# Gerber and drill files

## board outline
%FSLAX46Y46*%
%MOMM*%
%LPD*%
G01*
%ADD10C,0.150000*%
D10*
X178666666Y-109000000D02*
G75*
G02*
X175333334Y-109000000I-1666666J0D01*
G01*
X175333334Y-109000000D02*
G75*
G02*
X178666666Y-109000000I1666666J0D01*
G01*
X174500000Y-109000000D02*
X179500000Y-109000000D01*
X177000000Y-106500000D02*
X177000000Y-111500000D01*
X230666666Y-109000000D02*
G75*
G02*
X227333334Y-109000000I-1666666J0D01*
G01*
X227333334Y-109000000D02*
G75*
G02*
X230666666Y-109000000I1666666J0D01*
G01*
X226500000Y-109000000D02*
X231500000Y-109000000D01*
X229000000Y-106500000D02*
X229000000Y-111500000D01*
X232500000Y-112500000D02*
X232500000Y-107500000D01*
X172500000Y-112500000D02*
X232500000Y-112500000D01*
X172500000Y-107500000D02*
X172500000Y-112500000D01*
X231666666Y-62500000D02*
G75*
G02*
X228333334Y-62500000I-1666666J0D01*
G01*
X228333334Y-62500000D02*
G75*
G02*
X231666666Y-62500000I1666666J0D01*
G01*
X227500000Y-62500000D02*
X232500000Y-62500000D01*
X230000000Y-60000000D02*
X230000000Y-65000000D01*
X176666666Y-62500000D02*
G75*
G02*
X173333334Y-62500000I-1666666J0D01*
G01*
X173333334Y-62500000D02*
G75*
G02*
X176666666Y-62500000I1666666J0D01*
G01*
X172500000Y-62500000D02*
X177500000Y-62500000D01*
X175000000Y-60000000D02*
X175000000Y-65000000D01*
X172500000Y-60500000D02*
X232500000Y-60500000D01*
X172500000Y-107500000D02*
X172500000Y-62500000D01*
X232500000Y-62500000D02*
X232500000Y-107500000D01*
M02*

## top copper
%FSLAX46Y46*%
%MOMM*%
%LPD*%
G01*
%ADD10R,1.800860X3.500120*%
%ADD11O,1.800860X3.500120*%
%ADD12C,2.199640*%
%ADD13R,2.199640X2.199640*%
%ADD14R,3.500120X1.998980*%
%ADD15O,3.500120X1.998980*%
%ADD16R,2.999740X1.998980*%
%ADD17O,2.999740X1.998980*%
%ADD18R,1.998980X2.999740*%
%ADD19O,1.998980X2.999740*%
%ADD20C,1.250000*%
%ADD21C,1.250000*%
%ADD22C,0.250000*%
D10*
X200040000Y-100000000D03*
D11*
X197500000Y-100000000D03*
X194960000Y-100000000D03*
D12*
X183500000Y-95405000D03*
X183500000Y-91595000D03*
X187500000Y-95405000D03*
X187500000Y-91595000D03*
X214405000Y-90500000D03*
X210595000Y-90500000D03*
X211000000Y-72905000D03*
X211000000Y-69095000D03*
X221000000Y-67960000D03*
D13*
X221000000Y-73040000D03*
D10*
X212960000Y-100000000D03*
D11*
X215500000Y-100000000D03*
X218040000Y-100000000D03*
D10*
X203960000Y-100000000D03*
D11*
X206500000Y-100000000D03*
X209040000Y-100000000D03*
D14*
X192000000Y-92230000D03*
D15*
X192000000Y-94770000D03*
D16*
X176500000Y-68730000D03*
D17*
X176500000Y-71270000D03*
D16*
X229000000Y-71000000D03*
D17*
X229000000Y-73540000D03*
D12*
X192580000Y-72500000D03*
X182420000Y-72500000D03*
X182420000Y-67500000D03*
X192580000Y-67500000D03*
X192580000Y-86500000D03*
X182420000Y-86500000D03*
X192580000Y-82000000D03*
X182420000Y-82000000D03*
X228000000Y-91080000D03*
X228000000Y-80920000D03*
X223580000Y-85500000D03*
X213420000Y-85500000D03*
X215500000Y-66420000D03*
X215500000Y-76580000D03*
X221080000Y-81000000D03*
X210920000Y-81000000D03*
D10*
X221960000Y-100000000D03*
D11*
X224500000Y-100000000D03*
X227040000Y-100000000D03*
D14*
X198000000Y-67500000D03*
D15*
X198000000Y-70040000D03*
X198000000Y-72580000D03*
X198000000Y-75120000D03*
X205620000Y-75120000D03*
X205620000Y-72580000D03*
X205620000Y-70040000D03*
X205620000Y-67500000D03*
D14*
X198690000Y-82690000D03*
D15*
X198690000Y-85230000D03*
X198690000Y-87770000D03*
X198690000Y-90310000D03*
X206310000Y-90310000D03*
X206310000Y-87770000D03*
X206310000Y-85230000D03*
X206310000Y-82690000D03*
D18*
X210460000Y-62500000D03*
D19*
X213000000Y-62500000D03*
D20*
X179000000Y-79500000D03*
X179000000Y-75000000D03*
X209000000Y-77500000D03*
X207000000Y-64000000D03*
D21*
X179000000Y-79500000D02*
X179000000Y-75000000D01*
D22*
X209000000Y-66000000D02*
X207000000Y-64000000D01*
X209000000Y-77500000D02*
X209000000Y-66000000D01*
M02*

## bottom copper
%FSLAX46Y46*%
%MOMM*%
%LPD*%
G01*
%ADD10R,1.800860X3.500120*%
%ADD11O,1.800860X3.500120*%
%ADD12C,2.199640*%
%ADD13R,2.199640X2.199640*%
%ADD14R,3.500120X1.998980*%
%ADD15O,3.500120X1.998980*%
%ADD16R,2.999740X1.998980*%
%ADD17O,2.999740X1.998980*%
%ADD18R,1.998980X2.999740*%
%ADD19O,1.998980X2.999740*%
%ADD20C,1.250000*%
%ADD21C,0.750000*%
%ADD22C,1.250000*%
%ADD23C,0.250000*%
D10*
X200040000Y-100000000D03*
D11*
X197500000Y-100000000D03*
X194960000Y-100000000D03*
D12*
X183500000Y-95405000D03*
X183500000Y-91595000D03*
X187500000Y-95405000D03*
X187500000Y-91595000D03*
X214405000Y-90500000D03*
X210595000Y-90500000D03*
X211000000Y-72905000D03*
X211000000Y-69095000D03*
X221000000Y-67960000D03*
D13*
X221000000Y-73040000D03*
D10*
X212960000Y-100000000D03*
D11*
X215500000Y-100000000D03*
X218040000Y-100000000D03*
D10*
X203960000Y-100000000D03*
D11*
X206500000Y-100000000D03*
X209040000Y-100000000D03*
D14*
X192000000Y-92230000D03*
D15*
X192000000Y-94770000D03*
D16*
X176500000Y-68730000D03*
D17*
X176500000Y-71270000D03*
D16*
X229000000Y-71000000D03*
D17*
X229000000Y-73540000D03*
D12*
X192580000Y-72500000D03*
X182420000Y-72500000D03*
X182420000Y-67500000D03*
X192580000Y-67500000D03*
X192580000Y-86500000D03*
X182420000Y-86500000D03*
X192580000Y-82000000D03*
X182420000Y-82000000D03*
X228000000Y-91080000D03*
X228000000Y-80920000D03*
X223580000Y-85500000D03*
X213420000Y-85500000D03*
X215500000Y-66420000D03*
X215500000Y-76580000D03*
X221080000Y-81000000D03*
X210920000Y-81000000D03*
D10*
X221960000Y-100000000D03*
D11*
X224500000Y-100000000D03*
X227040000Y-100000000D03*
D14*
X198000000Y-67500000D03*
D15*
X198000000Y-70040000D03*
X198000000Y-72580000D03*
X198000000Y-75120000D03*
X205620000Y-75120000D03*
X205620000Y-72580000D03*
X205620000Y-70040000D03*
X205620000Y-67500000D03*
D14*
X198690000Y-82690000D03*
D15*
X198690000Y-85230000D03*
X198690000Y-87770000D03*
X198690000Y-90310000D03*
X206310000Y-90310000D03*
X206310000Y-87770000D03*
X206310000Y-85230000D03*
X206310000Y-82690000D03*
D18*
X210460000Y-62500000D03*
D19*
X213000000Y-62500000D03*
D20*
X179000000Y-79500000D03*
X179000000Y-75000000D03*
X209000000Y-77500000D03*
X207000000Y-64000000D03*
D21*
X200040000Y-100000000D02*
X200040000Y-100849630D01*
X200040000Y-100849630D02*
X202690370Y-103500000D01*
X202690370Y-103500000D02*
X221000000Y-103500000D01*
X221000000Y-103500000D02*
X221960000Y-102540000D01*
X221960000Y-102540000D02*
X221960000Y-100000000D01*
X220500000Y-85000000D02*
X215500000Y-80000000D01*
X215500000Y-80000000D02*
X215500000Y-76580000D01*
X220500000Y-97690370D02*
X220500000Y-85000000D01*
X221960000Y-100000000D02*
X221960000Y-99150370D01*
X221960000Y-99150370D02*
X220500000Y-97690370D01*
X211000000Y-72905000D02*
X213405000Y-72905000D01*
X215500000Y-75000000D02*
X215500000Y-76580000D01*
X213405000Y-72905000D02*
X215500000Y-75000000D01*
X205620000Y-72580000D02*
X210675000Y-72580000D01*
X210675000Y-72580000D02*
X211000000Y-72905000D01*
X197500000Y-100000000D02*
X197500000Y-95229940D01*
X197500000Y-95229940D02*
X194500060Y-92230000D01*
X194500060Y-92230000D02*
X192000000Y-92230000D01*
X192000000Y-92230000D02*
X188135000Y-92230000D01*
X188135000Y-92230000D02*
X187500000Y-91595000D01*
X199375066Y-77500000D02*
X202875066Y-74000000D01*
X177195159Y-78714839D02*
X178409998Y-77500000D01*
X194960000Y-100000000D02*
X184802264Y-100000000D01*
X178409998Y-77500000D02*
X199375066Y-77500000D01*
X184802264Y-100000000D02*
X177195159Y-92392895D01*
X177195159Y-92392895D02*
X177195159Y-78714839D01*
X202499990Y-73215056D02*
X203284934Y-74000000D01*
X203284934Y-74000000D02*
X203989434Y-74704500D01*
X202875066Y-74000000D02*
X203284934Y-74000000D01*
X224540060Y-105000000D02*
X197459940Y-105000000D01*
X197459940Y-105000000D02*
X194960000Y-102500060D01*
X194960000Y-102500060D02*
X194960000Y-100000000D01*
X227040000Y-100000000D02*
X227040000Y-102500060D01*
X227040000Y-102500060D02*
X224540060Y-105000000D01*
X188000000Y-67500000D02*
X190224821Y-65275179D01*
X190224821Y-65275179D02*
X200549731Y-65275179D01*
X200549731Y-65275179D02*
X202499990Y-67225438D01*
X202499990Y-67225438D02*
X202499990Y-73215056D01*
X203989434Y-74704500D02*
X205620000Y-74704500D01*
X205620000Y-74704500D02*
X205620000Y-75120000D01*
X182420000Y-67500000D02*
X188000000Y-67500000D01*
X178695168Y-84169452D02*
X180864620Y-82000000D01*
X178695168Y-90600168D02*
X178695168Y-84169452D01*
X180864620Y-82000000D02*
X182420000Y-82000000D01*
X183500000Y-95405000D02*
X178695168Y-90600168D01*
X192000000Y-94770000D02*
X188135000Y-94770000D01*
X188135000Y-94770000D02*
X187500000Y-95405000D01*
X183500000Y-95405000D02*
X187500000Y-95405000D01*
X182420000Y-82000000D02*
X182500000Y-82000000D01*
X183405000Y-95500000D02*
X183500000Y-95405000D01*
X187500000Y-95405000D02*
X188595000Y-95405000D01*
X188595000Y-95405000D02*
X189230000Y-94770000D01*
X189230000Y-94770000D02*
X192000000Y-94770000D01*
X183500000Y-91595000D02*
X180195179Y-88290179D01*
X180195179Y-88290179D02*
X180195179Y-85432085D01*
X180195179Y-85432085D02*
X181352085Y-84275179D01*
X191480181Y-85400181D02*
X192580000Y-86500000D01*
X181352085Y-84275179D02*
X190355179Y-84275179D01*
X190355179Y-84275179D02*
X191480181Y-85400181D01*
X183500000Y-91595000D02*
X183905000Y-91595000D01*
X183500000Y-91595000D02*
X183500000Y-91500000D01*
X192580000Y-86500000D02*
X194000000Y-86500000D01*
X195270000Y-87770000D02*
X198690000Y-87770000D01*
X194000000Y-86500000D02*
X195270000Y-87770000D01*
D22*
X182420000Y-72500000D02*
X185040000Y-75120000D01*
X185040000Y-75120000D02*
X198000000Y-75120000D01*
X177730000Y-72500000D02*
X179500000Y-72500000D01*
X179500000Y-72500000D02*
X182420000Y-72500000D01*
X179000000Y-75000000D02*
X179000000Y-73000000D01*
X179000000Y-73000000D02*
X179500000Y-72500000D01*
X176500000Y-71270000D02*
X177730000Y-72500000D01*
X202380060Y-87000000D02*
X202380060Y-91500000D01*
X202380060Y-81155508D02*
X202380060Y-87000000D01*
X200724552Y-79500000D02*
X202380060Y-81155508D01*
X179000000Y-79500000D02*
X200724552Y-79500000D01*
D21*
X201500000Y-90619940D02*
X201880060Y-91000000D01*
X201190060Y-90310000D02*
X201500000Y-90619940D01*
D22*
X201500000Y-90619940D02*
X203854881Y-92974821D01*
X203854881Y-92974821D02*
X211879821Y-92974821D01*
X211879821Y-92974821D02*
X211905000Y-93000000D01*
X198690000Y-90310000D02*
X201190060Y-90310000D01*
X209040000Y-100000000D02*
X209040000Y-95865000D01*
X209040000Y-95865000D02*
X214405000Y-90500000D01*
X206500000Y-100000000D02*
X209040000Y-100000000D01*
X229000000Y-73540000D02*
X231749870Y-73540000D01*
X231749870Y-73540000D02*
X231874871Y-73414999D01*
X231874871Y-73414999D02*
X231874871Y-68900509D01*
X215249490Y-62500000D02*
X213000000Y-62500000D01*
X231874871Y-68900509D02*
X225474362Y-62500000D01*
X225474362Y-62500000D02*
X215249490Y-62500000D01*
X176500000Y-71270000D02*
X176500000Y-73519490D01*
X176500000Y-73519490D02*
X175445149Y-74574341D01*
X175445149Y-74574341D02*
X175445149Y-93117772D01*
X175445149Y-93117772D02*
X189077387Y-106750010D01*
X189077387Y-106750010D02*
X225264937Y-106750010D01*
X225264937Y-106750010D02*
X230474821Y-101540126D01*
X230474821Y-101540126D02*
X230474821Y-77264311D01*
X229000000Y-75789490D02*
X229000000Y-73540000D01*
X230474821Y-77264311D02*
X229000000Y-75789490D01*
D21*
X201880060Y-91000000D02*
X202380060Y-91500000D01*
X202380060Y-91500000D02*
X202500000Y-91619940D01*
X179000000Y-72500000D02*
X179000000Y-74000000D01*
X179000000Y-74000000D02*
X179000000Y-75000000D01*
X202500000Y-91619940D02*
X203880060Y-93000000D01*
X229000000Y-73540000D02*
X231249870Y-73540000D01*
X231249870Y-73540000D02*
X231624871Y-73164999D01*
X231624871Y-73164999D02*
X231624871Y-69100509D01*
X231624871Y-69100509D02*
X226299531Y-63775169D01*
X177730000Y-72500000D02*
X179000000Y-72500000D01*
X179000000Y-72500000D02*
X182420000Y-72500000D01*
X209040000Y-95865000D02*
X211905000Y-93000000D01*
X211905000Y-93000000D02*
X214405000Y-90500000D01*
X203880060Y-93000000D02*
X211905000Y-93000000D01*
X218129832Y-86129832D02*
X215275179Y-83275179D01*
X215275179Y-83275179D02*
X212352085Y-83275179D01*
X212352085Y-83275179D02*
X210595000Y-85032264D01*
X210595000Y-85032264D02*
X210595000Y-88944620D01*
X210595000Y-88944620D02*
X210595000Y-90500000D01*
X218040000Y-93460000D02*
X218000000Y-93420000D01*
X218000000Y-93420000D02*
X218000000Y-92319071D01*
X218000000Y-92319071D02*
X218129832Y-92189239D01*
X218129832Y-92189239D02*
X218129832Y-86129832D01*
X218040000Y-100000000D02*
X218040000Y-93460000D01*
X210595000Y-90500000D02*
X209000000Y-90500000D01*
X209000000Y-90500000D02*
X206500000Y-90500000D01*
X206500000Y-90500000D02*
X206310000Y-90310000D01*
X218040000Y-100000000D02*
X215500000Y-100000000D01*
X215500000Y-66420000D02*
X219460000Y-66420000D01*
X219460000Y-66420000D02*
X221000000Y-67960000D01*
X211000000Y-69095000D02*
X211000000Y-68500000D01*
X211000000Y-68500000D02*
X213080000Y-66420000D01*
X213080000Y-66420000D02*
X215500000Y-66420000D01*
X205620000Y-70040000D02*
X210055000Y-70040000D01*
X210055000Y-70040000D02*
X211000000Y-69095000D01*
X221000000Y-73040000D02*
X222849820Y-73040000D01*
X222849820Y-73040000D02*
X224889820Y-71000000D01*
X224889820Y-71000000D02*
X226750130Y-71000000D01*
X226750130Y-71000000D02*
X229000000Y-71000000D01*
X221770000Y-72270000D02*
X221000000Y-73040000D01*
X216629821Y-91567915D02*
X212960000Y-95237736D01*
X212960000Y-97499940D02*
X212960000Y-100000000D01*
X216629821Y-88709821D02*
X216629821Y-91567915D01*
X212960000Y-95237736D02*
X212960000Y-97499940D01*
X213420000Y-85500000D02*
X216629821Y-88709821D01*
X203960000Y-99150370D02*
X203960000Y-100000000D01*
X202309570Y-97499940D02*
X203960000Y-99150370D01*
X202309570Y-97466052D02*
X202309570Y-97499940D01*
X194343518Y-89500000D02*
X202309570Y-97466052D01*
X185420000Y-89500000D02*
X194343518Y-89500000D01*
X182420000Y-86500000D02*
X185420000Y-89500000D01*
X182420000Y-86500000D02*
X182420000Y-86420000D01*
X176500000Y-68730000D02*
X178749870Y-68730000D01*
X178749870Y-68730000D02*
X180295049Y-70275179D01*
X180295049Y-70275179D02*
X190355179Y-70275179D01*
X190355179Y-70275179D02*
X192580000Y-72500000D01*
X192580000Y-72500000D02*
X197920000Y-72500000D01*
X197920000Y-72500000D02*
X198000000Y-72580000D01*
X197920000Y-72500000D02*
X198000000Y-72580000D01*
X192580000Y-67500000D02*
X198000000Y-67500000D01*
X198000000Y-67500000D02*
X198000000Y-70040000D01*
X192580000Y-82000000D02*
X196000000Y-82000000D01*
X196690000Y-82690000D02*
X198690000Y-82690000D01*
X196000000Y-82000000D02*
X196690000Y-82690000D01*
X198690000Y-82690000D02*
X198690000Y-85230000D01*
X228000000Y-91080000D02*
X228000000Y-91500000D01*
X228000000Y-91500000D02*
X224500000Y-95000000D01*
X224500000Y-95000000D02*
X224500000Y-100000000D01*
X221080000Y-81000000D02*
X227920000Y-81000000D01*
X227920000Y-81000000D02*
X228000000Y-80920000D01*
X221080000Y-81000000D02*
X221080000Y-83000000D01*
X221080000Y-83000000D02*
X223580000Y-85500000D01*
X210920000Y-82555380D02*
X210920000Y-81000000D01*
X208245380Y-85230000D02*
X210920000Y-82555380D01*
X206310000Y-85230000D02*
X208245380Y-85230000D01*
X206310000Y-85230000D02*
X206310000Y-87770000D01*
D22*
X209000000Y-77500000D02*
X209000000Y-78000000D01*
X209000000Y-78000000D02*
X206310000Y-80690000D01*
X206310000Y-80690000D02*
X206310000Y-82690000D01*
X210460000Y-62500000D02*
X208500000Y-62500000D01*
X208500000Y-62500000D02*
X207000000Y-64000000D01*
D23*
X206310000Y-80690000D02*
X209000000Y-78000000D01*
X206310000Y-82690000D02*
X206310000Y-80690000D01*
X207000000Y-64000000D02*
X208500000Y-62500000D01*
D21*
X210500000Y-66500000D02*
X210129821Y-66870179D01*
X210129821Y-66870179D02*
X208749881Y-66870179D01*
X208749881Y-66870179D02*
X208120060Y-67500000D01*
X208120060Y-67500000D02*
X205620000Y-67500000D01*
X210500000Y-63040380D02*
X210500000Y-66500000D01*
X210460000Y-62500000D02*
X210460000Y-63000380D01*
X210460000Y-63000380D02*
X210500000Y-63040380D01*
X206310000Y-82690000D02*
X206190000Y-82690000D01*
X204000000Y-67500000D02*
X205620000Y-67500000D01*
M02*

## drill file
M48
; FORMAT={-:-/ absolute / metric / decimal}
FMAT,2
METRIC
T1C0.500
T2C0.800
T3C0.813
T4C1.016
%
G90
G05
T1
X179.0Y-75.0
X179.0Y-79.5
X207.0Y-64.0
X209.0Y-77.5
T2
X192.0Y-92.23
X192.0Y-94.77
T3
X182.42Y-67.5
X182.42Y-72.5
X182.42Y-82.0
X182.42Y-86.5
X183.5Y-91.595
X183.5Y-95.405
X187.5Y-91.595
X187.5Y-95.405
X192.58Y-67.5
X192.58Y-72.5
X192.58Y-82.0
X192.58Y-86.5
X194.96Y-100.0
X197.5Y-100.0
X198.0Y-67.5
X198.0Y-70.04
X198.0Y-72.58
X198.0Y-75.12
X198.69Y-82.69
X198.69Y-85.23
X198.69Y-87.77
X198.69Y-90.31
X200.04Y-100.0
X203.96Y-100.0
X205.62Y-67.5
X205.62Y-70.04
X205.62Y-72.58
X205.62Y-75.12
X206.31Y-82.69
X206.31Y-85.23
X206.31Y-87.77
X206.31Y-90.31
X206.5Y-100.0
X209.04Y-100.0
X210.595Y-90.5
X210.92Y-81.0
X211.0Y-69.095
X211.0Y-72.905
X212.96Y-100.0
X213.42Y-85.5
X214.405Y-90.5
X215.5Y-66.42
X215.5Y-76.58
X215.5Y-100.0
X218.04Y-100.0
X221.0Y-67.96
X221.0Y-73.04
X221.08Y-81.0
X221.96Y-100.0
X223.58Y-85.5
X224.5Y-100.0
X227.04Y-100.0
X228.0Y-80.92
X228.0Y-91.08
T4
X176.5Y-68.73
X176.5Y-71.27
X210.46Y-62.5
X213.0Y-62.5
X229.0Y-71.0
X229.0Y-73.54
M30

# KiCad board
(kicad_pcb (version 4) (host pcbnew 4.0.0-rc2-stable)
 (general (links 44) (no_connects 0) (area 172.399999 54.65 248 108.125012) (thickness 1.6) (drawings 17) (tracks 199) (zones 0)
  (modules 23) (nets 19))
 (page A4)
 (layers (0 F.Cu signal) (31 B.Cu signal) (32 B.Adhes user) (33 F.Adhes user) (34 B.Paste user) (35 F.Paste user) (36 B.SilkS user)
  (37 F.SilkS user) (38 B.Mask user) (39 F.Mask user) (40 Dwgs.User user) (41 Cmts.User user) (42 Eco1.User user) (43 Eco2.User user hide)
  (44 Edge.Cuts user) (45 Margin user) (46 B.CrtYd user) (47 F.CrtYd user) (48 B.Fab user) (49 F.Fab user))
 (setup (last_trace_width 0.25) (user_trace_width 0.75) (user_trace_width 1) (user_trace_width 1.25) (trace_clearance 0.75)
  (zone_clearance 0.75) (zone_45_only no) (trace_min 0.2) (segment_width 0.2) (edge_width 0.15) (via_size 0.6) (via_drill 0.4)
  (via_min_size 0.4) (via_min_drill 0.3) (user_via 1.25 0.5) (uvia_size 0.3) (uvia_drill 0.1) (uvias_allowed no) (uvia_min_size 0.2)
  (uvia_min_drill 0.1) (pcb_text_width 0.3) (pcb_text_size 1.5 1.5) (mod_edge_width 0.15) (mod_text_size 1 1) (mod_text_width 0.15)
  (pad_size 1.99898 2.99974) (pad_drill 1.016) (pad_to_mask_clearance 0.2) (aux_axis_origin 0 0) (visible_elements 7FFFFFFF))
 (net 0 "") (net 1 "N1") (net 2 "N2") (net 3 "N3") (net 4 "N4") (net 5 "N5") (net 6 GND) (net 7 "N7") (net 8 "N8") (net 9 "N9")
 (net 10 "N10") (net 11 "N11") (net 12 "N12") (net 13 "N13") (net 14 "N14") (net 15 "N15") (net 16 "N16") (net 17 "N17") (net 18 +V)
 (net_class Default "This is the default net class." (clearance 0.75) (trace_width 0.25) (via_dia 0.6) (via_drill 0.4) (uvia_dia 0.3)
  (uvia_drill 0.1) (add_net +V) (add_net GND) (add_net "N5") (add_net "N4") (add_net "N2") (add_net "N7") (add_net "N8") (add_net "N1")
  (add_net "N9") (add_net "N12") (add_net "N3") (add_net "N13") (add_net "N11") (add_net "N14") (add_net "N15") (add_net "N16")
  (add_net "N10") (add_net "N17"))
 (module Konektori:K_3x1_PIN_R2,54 (layer F.Cu) (at 197.5 100 180)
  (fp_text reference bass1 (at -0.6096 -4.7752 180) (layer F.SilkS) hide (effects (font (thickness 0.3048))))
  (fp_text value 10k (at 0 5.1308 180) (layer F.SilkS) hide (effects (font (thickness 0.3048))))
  (pad 1 thru_hole rect (at -2.54 0 180) (size 1.80086 3.50012) (drill 0.8128) (layers *.Cu *.Mask) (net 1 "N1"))
  (pad 2 thru_hole oval (at 0 0 180) (size 1.80086 3.50012) (drill 0.8128) (layers *.Cu *.Mask) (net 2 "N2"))
  (pad 3 thru_hole oval (at 2.54 0 180) (size 1.80086 3.50012) (drill 0.8128) (layers *.Cu *.Mask) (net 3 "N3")))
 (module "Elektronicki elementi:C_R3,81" (layer F.Cu) (at 183.5 93.5 270)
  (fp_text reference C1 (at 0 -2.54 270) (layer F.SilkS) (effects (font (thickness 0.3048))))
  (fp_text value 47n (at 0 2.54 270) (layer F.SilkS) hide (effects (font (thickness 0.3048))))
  (pad 2 thru_hole circle (at 1.905 0 270) (size 2.19964 2.19964) (drill 0.8128) (layers *.Cu) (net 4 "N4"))
  (pad 1 thru_hole circle (at -1.905 0 270) (size 2.19964 2.19964) (drill 0.8128) (layers *.Cu) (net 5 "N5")))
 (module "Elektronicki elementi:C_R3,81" (layer F.Cu) (at 187.5 93.5 270)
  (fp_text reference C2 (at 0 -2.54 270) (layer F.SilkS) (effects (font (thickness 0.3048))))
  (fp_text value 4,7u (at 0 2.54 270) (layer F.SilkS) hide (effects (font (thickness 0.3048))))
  (pad 2 thru_hole circle (at 1.905 0 270) (size 2.19964 2.19964) (drill 0.8128) (layers *.Cu) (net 4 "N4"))
  (pad 1 thru_hole circle (at -1.905 0 270) (size 2.19964 2.19964) (drill 0.8128) (layers *.Cu) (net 2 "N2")))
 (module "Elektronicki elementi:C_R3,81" (layer F.Cu) (at 212.5 90.5)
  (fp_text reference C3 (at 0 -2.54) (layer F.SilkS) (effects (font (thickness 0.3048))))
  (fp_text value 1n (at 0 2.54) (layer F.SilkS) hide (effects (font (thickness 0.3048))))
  (pad 2 thru_hole circle (at 1.905 0) (size 2.19964 2.19964) (drill 0.8128) (layers *.Cu) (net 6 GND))
  (pad 1 thru_hole circle (at -1.905 0) (size 2.19964 2.19964) (drill 0.8128) (layers *.Cu) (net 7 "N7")))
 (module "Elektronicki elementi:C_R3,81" (layer F.Cu) (at 211 71 270)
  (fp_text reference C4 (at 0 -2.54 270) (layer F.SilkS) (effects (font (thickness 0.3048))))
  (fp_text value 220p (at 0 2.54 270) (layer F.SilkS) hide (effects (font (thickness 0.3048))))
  (pad 2 thru_hole circle (at 1.905 0 270) (size 2.19964 2.19964) (drill 0.8128) (layers *.Cu) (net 1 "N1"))
  (pad 1 thru_hole circle (at -1.905 0 270) (size 2.19964 2.19964) (drill 0.8128) (layers *.Cu) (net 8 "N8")))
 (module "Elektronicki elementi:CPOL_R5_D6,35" (layer F.Cu) (at 221 70.5 270)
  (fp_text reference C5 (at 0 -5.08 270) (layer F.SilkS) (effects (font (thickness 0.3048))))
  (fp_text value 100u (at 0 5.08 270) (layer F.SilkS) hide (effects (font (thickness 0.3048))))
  (pad + thru_hole circle (at -2.54 0 270) (size 2.19964 2.19964) (drill 0.8128) (layers *.Cu) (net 8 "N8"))
  (pad - thru_hole rect (at 2.54 0 270) (size 2.19964 2.19964) (drill 0.8128) (layers *.Cu) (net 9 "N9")))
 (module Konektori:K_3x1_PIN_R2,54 (layer F.Cu) (at 215.5 100)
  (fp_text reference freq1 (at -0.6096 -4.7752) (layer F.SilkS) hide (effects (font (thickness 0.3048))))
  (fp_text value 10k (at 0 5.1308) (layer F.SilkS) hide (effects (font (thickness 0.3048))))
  (pad 1 thru_hole rect (at -2.54 0) (size 1.80086 3.50012) (drill 0.8128) (layers *.Cu *.Mask) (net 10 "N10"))
  (pad 2 thru_hole oval (at 0 0) (size 1.80086 3.50012) (drill 0.8128) (layers *.Cu *.Mask) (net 7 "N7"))
  (pad 3 thru_hole oval (at 2.54 0) (size 1.80086 3.50012) (drill 0.8128) (layers *.Cu *.Mask) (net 7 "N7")))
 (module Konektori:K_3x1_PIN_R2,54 (layer F.Cu) (at 206.5 100)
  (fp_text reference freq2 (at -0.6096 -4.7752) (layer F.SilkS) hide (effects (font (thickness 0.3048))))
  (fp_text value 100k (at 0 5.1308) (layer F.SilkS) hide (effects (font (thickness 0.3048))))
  (pad 1 thru_hole rect (at -2.54 0) (size 1.80086 3.50012) (drill 0.8128) (layers *.Cu *.Mask) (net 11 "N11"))
  (pad 2 thru_hole oval (at 0 0) (size 1.80086 3.50012) (drill 0.8128) (layers *.Cu *.Mask) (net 6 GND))
  (pad 3 thru_hole oval (at 2.54 0) (size 1.80086 3.50012) (drill 0.8128) (layers *.Cu *.Mask) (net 6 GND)))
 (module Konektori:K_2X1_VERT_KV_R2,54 (layer F.Cu) (at 192 93.5 270)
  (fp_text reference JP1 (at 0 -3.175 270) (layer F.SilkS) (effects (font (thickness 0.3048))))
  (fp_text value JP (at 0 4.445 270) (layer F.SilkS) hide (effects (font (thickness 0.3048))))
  (pad 1 thru_hole rect (at -1.27 0 270) (size 1.99898 3.50012) (drill 0.8001) (layers *.Cu) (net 2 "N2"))
  (pad 2 thru_hole oval (at 1.27 0 270) (size 1.99898 3.50012) (drill 0.8001) (layers *.Cu) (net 4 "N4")))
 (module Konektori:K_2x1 (layer F.Cu) (at 176.5 70 270)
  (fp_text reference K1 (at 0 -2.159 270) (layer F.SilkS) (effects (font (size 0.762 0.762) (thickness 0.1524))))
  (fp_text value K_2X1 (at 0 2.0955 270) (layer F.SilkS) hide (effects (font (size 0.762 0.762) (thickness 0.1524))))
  (pad 1 thru_hole rect (at -1.27 0 270) (size 1.99898 2.99974) (drill 1.016) (layers *.Cu *.Mask) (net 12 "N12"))
  (pad 2 thru_hole oval (at 1.27 0 270) (size 1.99898 2.99974) (drill 1.016) (layers *.Cu *.Mask) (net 6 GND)))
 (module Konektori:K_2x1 (layer F.Cu) (at 229 72.27 270)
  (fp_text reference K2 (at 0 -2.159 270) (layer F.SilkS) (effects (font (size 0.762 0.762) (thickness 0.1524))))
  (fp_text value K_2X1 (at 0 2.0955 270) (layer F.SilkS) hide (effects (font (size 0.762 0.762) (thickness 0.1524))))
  (pad 1 thru_hole rect (at -1.27 0 270) (size 1.99898 2.99974) (drill 1.016) (layers *.Cu *.Mask) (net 9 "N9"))
  (pad 2 thru_hole oval (at 1.27 0 270) (size 1.99898 2.99974) (drill 1.016) (layers *.Cu *.Mask) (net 6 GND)))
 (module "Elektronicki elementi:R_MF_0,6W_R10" (layer F.Cu) (at 187.5 72.5 180)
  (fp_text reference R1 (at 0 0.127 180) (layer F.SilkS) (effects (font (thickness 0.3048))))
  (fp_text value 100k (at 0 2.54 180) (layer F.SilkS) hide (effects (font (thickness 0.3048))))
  (pad 1 thru_hole circle (at -5.08 0 180) (size 2.19964 2.19964) (drill 0.8128) (layers *.Cu *.Mask) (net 12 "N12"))
  (pad 2 thru_hole circle (at 5.08 0 180) (size 2.19964 2.19964) (drill 0.8128) (layers *.Cu *.Mask) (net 6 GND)))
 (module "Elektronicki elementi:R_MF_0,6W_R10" (layer F.Cu) (at 187.5 67.5)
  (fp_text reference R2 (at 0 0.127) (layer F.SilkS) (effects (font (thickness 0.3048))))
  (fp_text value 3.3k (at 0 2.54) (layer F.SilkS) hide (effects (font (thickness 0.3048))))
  (pad 1 thru_hole circle (at -5.08 0) (size 2.19964 2.19964) (drill 0.8128) (layers *.Cu *.Mask) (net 3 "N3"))
  (pad 2 thru_hole circle (at 5.08 0) (size 2.19964 2.19964) (drill 0.8128) (layers *.Cu *.Mask) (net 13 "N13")))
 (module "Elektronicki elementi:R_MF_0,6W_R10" (layer F.Cu) (at 187.5 86.5 180)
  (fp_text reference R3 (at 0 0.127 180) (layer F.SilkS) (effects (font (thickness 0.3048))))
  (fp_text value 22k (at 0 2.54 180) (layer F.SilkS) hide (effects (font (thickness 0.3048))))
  (pad 1 thru_hole circle (at -5.08 0 180) (size 2.19964 2.19964) (drill 0.8128) (layers *.Cu *.Mask) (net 5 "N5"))
  (pad 2 thru_hole circle (at 5.08 0 180) (size 2.19964 2.19964) (drill 0.8128) (layers *.Cu *.Mask) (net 11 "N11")))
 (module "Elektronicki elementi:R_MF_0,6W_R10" (layer F.Cu) (at 187.5 82 180)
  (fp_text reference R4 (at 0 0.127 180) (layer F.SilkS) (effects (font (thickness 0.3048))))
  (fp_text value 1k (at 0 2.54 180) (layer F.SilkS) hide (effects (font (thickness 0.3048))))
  (pad 1 thru_hole circle (at -5.08 0 180) (size 2.19964 2.19964) (drill 0.8128) (layers *.Cu *.Mask) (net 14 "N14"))
  (pad 2 thru_hole circle (at 5.08 0 180) (size 2.19964 2.19964) (drill 0.8128) (layers *.Cu *.Mask) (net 4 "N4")))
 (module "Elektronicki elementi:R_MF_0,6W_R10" (layer F.Cu) (at 228 86 90)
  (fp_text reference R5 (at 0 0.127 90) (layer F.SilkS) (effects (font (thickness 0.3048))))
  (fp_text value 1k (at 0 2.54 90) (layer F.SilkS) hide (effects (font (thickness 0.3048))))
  (pad 1 thru_hole circle (at -5.08 0 90) (size 2.19964 2.19964) (drill 0.8128) (layers *.Cu *.Mask) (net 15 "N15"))
  (pad 2 thru_hole circle (at 5.08 0 90) (size 2.19964 2.19964) (drill 0.8128) (layers *.Cu *.Mask) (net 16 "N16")))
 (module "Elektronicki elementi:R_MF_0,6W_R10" (layer F.Cu) (at 218.5 85.5 180)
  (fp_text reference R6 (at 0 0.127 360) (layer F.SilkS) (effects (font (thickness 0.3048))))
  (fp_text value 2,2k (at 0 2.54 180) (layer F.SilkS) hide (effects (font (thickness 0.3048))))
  (pad 1 thru_hole circle (at -5.08 0 180) (size 2.19964 2.19964) (drill 0.8128) (layers *.Cu *.Mask) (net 16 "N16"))
  (pad 2 thru_hole circle (at 5.08 0 180) (size 2.19964 2.19964) (drill 0.8128) (layers *.Cu *.Mask) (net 10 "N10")))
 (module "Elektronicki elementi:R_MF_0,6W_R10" (layer F.Cu) (at 215.5 71.5 270)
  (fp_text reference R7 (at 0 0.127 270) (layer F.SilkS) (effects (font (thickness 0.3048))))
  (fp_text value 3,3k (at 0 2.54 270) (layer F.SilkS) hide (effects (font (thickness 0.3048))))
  (pad 1 thru_hole circle (at -5.08 0 270) (size 2.19964 2.19964) (drill 0.8128) (layers *.Cu *.Mask) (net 8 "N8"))
  (pad 2 thru_hole circle (at 5.08 0 270) (size 2.19964 2.19964) (drill 0.8128) (layers *.Cu *.Mask) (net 1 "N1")))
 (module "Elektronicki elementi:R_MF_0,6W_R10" (layer F.Cu) (at 216 81 180)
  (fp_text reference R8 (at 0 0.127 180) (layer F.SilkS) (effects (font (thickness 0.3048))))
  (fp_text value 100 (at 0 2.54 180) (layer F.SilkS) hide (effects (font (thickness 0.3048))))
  (pad 1 thru_hole circle (at -5.08 0 180) (size 2.19964 2.19964) (drill 0.8128) (layers *.Cu *.Mask) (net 16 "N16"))
  (pad 2 thru_hole circle (at 5.08 0 180) (size 2.19964 2.19964) (drill 0.8128) (layers *.Cu *.Mask) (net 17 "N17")))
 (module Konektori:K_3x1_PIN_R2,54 (layer F.Cu) (at 224.5 100)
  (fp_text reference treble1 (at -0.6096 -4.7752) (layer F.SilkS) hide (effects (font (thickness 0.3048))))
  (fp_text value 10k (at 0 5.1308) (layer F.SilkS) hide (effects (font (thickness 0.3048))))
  (pad 1 thru_hole rect (at -2.54 0) (size 1.80086 3.50012) (drill 0.8128) (layers *.Cu *.Mask) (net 1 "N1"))
  (pad 2 thru_hole oval (at 0 0) (size 1.80086 3.50012) (drill 0.8128) (layers *.Cu *.Mask) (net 15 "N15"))
  (pad 3 thru_hole oval (at 2.54 0) (size 1.80086 3.50012) (drill 0.8128) (layers *.Cu *.Mask) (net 3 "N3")))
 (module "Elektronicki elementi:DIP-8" (layer F.Cu) (at 201.81 71.31 270)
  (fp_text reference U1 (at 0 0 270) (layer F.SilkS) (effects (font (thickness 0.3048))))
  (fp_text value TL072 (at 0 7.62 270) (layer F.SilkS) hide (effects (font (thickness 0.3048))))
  (pad 1 thru_hole rect (at -3.81 3.81 270) (size 1.99898 3.50012) (drill 0.8128) (layers *.Cu) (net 13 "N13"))
  (pad 2 thru_hole oval (at -1.27 3.81 270) (size 1.99898 3.50012) (drill 0.8128) (layers *.Cu) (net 13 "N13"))
  (pad 3 thru_hole oval (at 1.27 3.81 270) (size 1.99898 3.50012) (drill 0.8128) (layers *.Cu) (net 12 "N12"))
  (pad 4 thru_hole oval (at 3.81 3.81 270) (size 1.99898 3.50012) (drill 0.8128) (layers *.Cu) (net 6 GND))
  (pad 5 thru_hole oval (at 3.81 -3.81 270) (size 1.99898 3.50012) (drill 0.8128) (layers *.Cu) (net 3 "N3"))
  (pad 6 thru_hole oval (at 1.27 -3.81 270) (size 1.99898 3.50012) (drill 0.8128) (layers *.Cu) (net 1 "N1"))
  (pad 7 thru_hole oval (at -1.27 -3.81 270) (size 1.99898 3.50012) (drill 0.8128) (layers *.Cu) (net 8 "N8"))
  (pad 8 thru_hole oval (at -3.81 -3.81 270) (size 1.99898 3.50012) (drill 0.8128) (layers *.Cu) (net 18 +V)))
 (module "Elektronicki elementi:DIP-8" (layer F.Cu) (at 202.5 86.5 270)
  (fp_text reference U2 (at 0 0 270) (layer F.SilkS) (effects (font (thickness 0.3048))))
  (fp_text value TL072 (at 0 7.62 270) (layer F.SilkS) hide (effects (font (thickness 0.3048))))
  (pad 1 thru_hole rect (at -3.81 3.81 270) (size 1.99898 3.50012) (drill 0.8128) (layers *.Cu) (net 14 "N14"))
  (pad 2 thru_hole oval (at -1.27 3.81 270) (size 1.99898 3.50012) (drill 0.8128) (layers *.Cu) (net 14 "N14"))
  (pad 3 thru_hole oval (at 1.27 3.81 270) (size 1.99898 3.50012) (drill 0.8128) (layers *.Cu) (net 5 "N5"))
  (pad 4 thru_hole oval (at 3.81 3.81 270) (size 1.99898 3.50012) (drill 0.8128) (layers *.Cu) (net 6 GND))
  (pad 5 thru_hole oval (at 3.81 -3.81 270) (size 1.99898 3.50012) (drill 0.8128) (layers *.Cu) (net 7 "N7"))
  (pad 6 thru_hole oval (at 1.27 -3.81 270) (size 1.99898 3.50012) (drill 0.8128) (layers *.Cu) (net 17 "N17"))
  (pad 7 thru_hole oval (at -1.27 -3.81 270) (size 1.99898 3.50012) (drill 0.8128) (layers *.Cu) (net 17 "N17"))
  (pad 8 thru_hole oval (at -3.81 -3.81 270) (size 1.99898 3.50012) (drill 0.8128) (layers *.Cu) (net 18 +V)))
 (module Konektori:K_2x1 (layer F.Cu) (at 211.73 62.5)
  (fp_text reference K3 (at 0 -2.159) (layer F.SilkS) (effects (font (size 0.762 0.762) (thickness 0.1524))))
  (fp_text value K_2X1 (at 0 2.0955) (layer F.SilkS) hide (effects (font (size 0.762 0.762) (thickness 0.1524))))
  (pad 1 thru_hole rect (at -1.27 0) (size 1.99898 2.99974) (drill 1.016) (layers *.Cu *.Mask) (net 18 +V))
  (pad 2 thru_hole oval (at 1.27 0) (size 1.99898 2.99974) (drill 1.016) (layers *.Cu *.Mask) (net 6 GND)))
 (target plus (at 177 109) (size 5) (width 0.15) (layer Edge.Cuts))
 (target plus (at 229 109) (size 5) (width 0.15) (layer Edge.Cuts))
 (gr_line (start 232.5 112.5) (end 232.5 107.5) (angle 90) (layer Edge.Cuts) (width 0.15))
 (gr_line (start 172.5 112.5) (end 232.5 112.5) (angle 90) (layer Edge.Cuts) (width 0.15))
 (gr_line (start 172.5 107.5) (end 172.5 112.5) (angle 90) (layer Edge.Cuts) (width 0.15))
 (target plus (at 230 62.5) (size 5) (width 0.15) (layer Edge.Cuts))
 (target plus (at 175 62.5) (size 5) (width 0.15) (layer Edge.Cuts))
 (gr_line (start 172.5 60.5) (end 232.5 60.5) (layer Edge.Cuts) (width 0.15))
 (gr_line (start 172.5 107.5) (end 172.5 62.5) (layer Edge.Cuts) (width 0.15))
 (gr_line (start 232.5 62.5) (end 232.5 107.5) (layer Edge.Cuts) (width 0.15))
 (segment (start 200.04 100) (end 200.04 100.84963) (width 0.75) (layer B.Cu) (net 1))
 (segment (start 200.04 100.84963) (end 202.69037 103.5) (width 0.75) (layer B.Cu) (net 1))
 (segment (start 202.69037 103.5) (end 221 103.5) (width 0.75) (layer B.Cu) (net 1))
 (segment (start 221 103.5) (end 221.96 102.54) (width 0.75) (layer B.Cu) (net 1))
 (segment (start 221.96 102.54) (end 221.96 100) (width 0.75) (layer B.Cu) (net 1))
 (segment (start 220.5 85) (end 215.5 80) (width 0.75) (layer B.Cu) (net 1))
 (segment (start 215.5 80) (end 215.5 76.58) (width 0.75) (layer B.Cu) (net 1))
 (segment (start 220.5 97.69037) (end 220.5 85) (width 0.75) (layer B.Cu) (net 1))
 (segment (start 221.96 100) (end 221.96 99.15037) (width 0.75) (layer B.Cu) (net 1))
 (segment (start 221.96 99.15037) (end 220.5 97.69037) (width 0.75) (layer B.Cu) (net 1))
 (segment (start 211 72.905) (end 213.405 72.905) (width 0.75) (layer B.Cu) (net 1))
 (segment (start 215.5 75) (end 215.5 76.58) (width 0.75) (layer B.Cu) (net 1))
 (segment (start 213.405 72.905) (end 215.5 75) (width 0.75) (layer B.Cu) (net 1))
 (segment (start 205.62 72.58) (end 210.675 72.58) (width 0.75) (layer B.Cu) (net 1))
 (segment (start 210.675 72.58) (end 211 72.905) (width 0.75) (layer B.Cu) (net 1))
 (segment (start 197.5 100) (end 197.5 95.22994) (width 0.75) (layer B.Cu) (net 2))
 (segment (start 197.5 95.22994) (end 194.50006 92.23) (width 0.75) (layer B.Cu) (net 2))
 (segment (start 194.50006 92.23) (end 192 92.23) (width 0.75) (layer B.Cu) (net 2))
 (segment (start 192 92.23) (end 188.135 92.23) (width 0.75) (layer B.Cu) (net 2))
 (segment (start 188.135 92.23) (end 187.5 91.595) (width 0.75) (layer B.Cu) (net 2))
 (segment (start 199.375066 77.5) (end 202.875066 74) (width 0.75) (layer B.Cu) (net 3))
 (segment (start 177.195159 78.714839) (end 178.409998 77.5) (width 0.75) (layer B.Cu) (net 3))
 (segment (start 194.96 100) (end 184.802264 100) (width 0.75) (layer B.Cu) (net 3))
 (segment (start 178.409998 77.5) (end 199.375066 77.5) (width 0.75) (layer B.Cu) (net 3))
 (segment (start 184.802264 100) (end 177.195159 92.392895) (width 0.75) (layer B.Cu) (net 3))
 (segment (start 177.195159 92.392895) (end 177.195159 78.714839) (width 0.75) (layer B.Cu) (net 3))
 (segment (start 202.49999 73.215056) (end 203.284934 74) (width 0.75) (layer B.Cu) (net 3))
 (segment (start 203.284934 74) (end 203.989434 74.7045) (width 0.75) (layer B.Cu) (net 3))
 (segment (start 202.875066 74) (end 203.284934 74) (width 0.75) (layer B.Cu) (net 3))
 (segment (start 224.54006 105) (end 197.45994 105) (width 0.75) (layer B.Cu) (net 3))
 (segment (start 197.45994 105) (end 194.96 102.50006) (width 0.75) (layer B.Cu) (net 3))
 (segment (start 194.96 102.50006) (end 194.96 100) (width 0.75) (layer B.Cu) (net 3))
 (segment (start 227.04 100) (end 227.04 102.50006) (width 0.75) (layer B.Cu) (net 3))
 (segment (start 227.04 102.50006) (end 224.54006 105) (width 0.75) (layer B.Cu) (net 3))
 (segment (start 188 67.5) (end 190.224821 65.275179) (width 0.75) (layer B.Cu) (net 3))
 (segment (start 190.224821 65.275179) (end 200.549731 65.275179) (width 0.75) (layer B.Cu) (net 3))
 (segment (start 200.549731 65.275179) (end 202.49999 67.225438) (width 0.75) (layer B.Cu) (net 3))
 (segment (start 202.49999 67.225438) (end 202.49999 73.215056) (width 0.75) (layer B.Cu) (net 3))
 (segment (start 203.989434 74.7045) (end 205.62 74.7045) (width 0.75) (layer B.Cu) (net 3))
 (segment (start 205.62 74.7045) (end 205.62 75.12) (width 0.75) (layer B.Cu) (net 3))
 (segment (start 182.42 67.5) (end 188 67.5) (width 0.75) (layer B.Cu) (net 3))
 (segment (start 178.695168 84.169452) (end 180.86462 82) (width 0.75) (layer B.Cu) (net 4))
 (segment (start 178.695168 90.600168) (end 178.695168 84.169452) (width 0.75) (layer B.Cu) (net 4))
 (segment (start 180.86462 82) (end 182.42 82) (width 0.75) (layer B.Cu) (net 4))
 (segment (start 183.5 95.405) (end 178.695168 90.600168) (width 0.75) (layer B.Cu) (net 4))
 (segment (start 192 94.77) (end 188.135 94.77) (width 0.75) (layer B.Cu) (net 4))
 (segment (start 188.135 94.77) (end 187.5 95.405) (width 0.75) (layer B.Cu) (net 4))
 (segment (start 183.5 95.405) (end 187.5 95.405) (width 0.75) (layer B.Cu) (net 4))
 (segment (start 182.42 82) (end 182.5 82) (width 0.75) (layer B.Cu) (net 4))
 (segment (start 183.405 95.5) (end 183.5 95.405) (width 0.75) (layer B.Cu) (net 4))
 (segment (start 187.5 95.405) (end 188.595 95.405) (width 0.75) (layer B.Cu) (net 4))
 (segment (start 188.595 95.405) (end 189.23 94.77) (width 0.75) (layer B.Cu) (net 4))
 (segment (start 189.23 94.77) (end 192 94.77) (width 0.75) (layer B.Cu) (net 4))
 (segment (start 183.5 91.595) (end 180.195179 88.290179) (width 0.75) (layer B.Cu) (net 5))
 (segment (start 180.195179 88.290179) (end 180.195179 85.432085) (width 0.75) (layer B.Cu) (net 5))
 (segment (start 180.195179 85.432085) (end 181.352085 84.275179) (width 0.75) (layer B.Cu) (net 5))
 (segment (start 191.480181 85.400181) (end 192.58 86.5) (width 0.75) (layer B.Cu) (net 5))
 (segment (start 181.352085 84.275179) (end 190.355179 84.275179) (width 0.75) (layer B.Cu) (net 5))
 (segment (start 190.355179 84.275179) (end 191.480181 85.400181) (width 0.75) (layer B.Cu) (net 5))
 (segment (start 183.5 91.595) (end 183.905 91.595) (width 0.75) (layer B.Cu) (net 5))
 (segment (start 183.5 91.595) (end 183.5 91.5) (width 0.75) (layer B.Cu) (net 5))
 (segment (start 192.58 86.5) (end 194 86.5) (width 0.75) (layer B.Cu) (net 5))
 (segment (start 195.27 87.77) (end 198.69 87.77) (width 0.75) (layer B.Cu) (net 5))
 (segment (start 194 86.5) (end 195.27 87.77) (width 0.75) (layer B.Cu) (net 5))
 (segment (start 179 79.5) (end 179 75) (width 1.25) (layer F.Cu) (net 6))
 (segment (start 182.42 72.5) (end 185.04 75.12) (width 1.25) (layer B.Cu) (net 6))
 (segment (start 185.04 75.12) (end 198 75.12) (width 1.25) (layer B.Cu) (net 6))
 (segment (start 177.73 72.5) (end 179.5 72.5) (width 1.25) (layer B.Cu) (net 6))
 (segment (start 179.5 72.5) (end 182.42 72.5) (width 1.25) (layer B.Cu) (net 6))
 (segment (start 179 75) (end 179 73) (width 1.25) (layer B.Cu) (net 6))
 (segment (start 179 73) (end 179.5 72.5) (width 1.25) (layer B.Cu) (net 6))
 (segment (start 176.5 71.27) (end 177.73 72.5) (width 1.25) (layer B.Cu) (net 6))
 (segment (start 202.38006 87) (end 202.38006 91.5) (width 1.25) (layer B.Cu) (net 6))
 (via (at 179 79.5) (size 1.25) (drill 0.5) (layers F.Cu B.Cu) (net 6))
 (segment (start 202.38006 81.155508) (end 202.38006 87) (width 1.25) (layer B.Cu) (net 6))
 (segment (start 200.724552 79.5) (end 202.38006 81.155508) (width 1.25) (layer B.Cu) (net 6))
 (segment (start 179 79.5) (end 200.724552 79.5) (width 1.25) (layer B.Cu) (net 6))
 (segment (start 201.5 90.61994) (end 201.88006 91) (width 0.75) (layer B.Cu) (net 6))
 (segment (start 201.19006 90.31) (end 201.5 90.61994) (width 0.75) (layer B.Cu) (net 6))
 (segment (start 201.5 90.61994) (end 203.854881 92.974821) (width 1.25) (layer B.Cu) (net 6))
 (segment (start 203.854881 92.974821) (end 211.879821 92.974821) (width 1.25) (layer B.Cu) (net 6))
 (segment (start 211.879821 92.974821) (end 211.905 93) (width 1.25) (layer B.Cu) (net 6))
 (segment (start 198.69 90.31) (end 201.19006 90.31) (width 1.25) (layer B.Cu) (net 6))
 (segment (start 209.04 100) (end 209.04 95.865) (width 1.25) (layer B.Cu) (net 6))
 (segment (start 209.04 95.865) (end 214.405 90.5) (width 1.25) (layer B.Cu) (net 6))
 (segment (start 206.5 100) (end 209.04 100) (width 1.25) (layer B.Cu) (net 6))
 (segment (start 229 73.54) (end 231.74987 73.54) (width 1.25) (layer B.Cu) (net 6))
 (segment (start 231.74987 73.54) (end 231.874871 73.414999) (width 1.25) (layer B.Cu) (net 6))
 (segment (start 231.874871 73.414999) (end 231.874871 68.900509) (width 1.25) (layer B.Cu) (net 6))
 (segment (start 215.24949 62.5) (end 213 62.5) (width 1.25) (layer B.Cu) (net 6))
 (segment (start 231.874871 68.900509) (end 225.474362 62.5) (width 1.25) (layer B.Cu) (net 6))
 (segment (start 225.474362 62.5) (end 215.24949 62.5) (width 1.25) (layer B.Cu) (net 6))
 (segment (start 176.5 71.27) (end 176.5 73.51949) (width 1.25) (layer B.Cu) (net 6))
 (segment (start 176.5 73.51949) (end 175.445149 74.574341) (width 1.25) (layer B.Cu) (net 6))
 (segment (start 175.445149 74.574341) (end 175.445149 93.117772) (width 1.25) (layer B.Cu) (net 6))
 (segment (start 175.445149 93.117772) (end 189.077387 106.75001) (width 1.25) (layer B.Cu) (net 6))
 (segment (start 189.077387 106.75001) (end 225.264937 106.75001) (width 1.25) (layer B.Cu) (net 6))
 (segment (start 225.264937 106.75001) (end 230.474821 101.540126) (width 1.25) (layer B.Cu) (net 6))
 (segment (start 230.474821 101.540126) (end 230.474821 77.264311) (width 1.25) (layer B.Cu) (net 6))
 (segment (start 229 75.78949) (end 229 73.54) (width 1.25) (layer B.Cu) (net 6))
 (segment (start 230.474821 77.264311) (end 229 75.78949) (width 1.25) (layer B.Cu) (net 6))
 (segment (start 201.88006 91) (end 202.38006 91.5) (width 0.75) (layer B.Cu) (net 6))
 (segment (start 202.38006 91.5) (end 202.5 91.61994) (width 0.75) (layer B.Cu) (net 6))
 (segment (start 179 72.5) (end 179 74) (width 0.75) (layer B.Cu) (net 6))
 (via (at 179 75) (size 1.25) (drill 0.5) (layers F.Cu B.Cu) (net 6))
 (segment (start 179 74) (end 179 75) (width 0.75) (layer B.Cu) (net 6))
 (segment (start 202.5 91.61994) (end 203.88006 93) (width 0.75) (layer B.Cu) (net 6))
 (segment (start 229 73.54) (end 231.24987 73.54) (width 0.75) (layer B.Cu) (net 6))
 (segment (start 231.24987 73.54) (end 231.624871 73.164999) (width 0.75) (layer B.Cu) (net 6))
 (segment (start 231.624871 73.164999) (end 231.624871 69.100509) (width 0.75) (layer B.Cu) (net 6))
 (segment (start 231.624871 69.100509) (end 226.299531 63.775169) (width 0.75) (layer B.Cu) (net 6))
 (segment (start 177.73 72.5) (end 179 72.5) (width 0.75) (layer B.Cu) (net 6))
 (segment (start 179 72.5) (end 182.42 72.5) (width 0.75) (layer B.Cu) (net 6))
 (segment (start 209.04 95.865) (end 211.905 93) (width 0.75) (layer B.Cu) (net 6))
 (segment (start 211.905 93) (end 214.405 90.5) (width 0.75) (layer B.Cu) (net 6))
 (segment (start 203.88006 93) (end 211.905 93) (width 0.75) (layer B.Cu) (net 6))
 (segment (start 218.129832 86.129832) (end 215.275179 83.275179) (width 0.75) (layer B.Cu) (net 7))
 (segment (start 215.275179 83.275179) (end 212.352085 83.275179) (width 0.75) (layer B.Cu) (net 7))
 (segment (start 212.352085 83.275179) (end 210.595 85.032264) (width 0.75) (layer B.Cu) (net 7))
 (segment (start 210.595 85.032264) (end 210.595 88.94462) (width 0.75) (layer B.Cu) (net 7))
 (segment (start 210.595 88.94462) (end 210.595 90.5) (width 0.75) (layer B.Cu) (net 7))
 (segment (start 218.04 93.46) (end 218 93.42) (width 0.75) (layer B.Cu) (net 7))
 (segment (start 218 93.42) (end 218 92.319071) (width 0.75) (layer B.Cu) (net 7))
 (segment (start 218 92.319071) (end 218.129832 92.189239) (width 0.75) (layer B.Cu) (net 7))
 (segment (start 218.129832 92.189239) (end 218.129832 86.129832) (width 0.75) (layer B.Cu) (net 7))
 (segment (start 218.04 100) (end 218.04 93.46) (width 0.75) (layer B.Cu) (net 7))
 (segment (start 210.595 90.5) (end 209 90.5) (width 0.75) (layer B.Cu) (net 7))
 (segment (start 209 90.5) (end 206.5 90.5) (width 0.75) (layer B.Cu) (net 7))
 (segment (start 206.5 90.5) (end 206.31 90.31) (width 0.75) (layer B.Cu) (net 7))
 (segment (start 218.04 100) (end 215.5 100) (width 0.75) (layer B.Cu) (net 7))
 (segment (start 215.5 66.42) (end 219.46 66.42) (width 0.75) (layer B.Cu) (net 8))
 (segment (start 219.46 66.42) (end 221 67.96) (width 0.75) (layer B.Cu) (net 8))
 (segment (start 211 69.095) (end 211 68.5) (width 0.75) (layer B.Cu) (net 8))
 (segment (start 211 68.5) (end 213.08 66.42) (width 0.75) (layer B.Cu) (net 8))
 (segment (start 213.08 66.42) (end 215.5 66.42) (width 0.75) (layer B.Cu) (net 8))
 (segment (start 205.62 70.04) (end 210.055 70.04) (width 0.75) (layer B.Cu) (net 8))
 (segment (start 210.055 70.04) (end 211 69.095) (width 0.75) (layer B.Cu) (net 8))
 (segment (start 221 73.04) (end 222.84982 73.04) (width 0.75) (layer B.Cu) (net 9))
 (segment (start 222.84982 73.04) (end 224.88982 71) (width 0.75) (layer B.Cu) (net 9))
 (segment (start 224.88982 71) (end 226.75013 71) (width 0.75) (layer B.Cu) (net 9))
 (segment (start 226.75013 71) (end 229 71) (width 0.75) (layer B.Cu) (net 9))
 (segment (start 221.77 72.27) (end 221 73.04) (width 0.75) (layer B.Cu) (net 9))
 (segment (start 216.629821 91.567915) (end 212.96 95.237736) (width 0.75) (layer B.Cu) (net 10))
 (segment (start 212.96 97.49994) (end 212.96 100) (width 0.75) (layer B.Cu) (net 10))
 (segment (start 216.629821 88.709821) (end 216.629821 91.567915) (width 0.75) (layer B.Cu) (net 10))
 (segment (start 212.96 95.237736) (end 212.96 97.49994) (width 0.75) (layer B.Cu) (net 10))
 (segment (start 213.42 85.5) (end 216.629821 88.709821) (width 0.75) (layer B.Cu) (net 10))
 (segment (start 203.96 99.15037) (end 203.96 100) (width 0.75) (layer B.Cu) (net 11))
 (segment (start 202.30957 97.49994) (end 203.96 99.15037) (width 0.75) (layer B.Cu) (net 11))
 (segment (start 202.30957 97.466052) (end 202.30957 97.49994) (width 0.75) (layer B.Cu) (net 11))
 (segment (start 194.343518 89.5) (end 202.30957 97.466052) (width 0.75) (layer B.Cu) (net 11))
 (segment (start 185.42 89.5) (end 194.343518 89.5) (width 0.75) (layer B.Cu) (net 11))
 (segment (start 182.42 86.5) (end 185.42 89.5) (width 0.75) (layer B.Cu) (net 11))
 (segment (start 182.42 86.5) (end 182.42 86.42) (width 0.75) (layer B.Cu) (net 11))
 (segment (start 176.5 68.73) (end 178.74987 68.73) (width 0.75) (layer B.Cu) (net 12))
 (segment (start 178.74987 68.73) (end 180.295049 70.275179) (width 0.75) (layer B.Cu) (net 12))
 (segment (start 180.295049 70.275179) (end 190.355179 70.275179) (width 0.75) (layer B.Cu) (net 12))
 (segment (start 190.355179 70.275179) (end 192.58 72.5) (width 0.75) (layer B.Cu) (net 12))
 (segment (start 192.58 72.5) (end 197.92 72.5) (width 0.75) (layer B.Cu) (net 12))
 (segment (start 197.92 72.5) (end 198 72.58) (width 0.75) (layer B.Cu) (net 12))
 (segment (start 197.92 72.5) (end 198 72.58) (width 0.75) (layer B.Cu) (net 12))
 (segment (start 192.58 67.5) (end 198 67.5) (width 0.75) (layer B.Cu) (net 13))
 (segment (start 198 67.5) (end 198 70.04) (width 0.75) (layer B.Cu) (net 13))
 (segment (start 192.58 82) (end 196 82) (width 0.75) (layer B.Cu) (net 14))
 (segment (start 196.69 82.69) (end 198.69 82.69) (width 0.75) (layer B.Cu) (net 14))
 (segment (start 196 82) (end 196.69 82.69) (width 0.75) (layer B.Cu) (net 14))
 (segment (start 198.69 82.69) (end 198.69 85.23) (width 0.75) (layer B.Cu) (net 14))
 (segment (start 228 91.08) (end 228 91.5) (width 0.75) (layer B.Cu) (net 15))
 (segment (start 228 91.5) (end 224.5 95) (width 0.75) (layer B.Cu) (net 15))
 (segment (start 224.5 95) (end 224.5 100) (width 0.75) (layer B.Cu) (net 15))
 (segment (start 221.08 81) (end 227.92 81) (width 0.75) (layer B.Cu) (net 16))
 (segment (start 227.92 81) (end 228 80.92) (width 0.75) (layer B.Cu) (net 16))
 (segment (start 221.08 81) (end 221.08 83) (width 0.75) (layer B.Cu) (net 16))
 (segment (start 221.08 83) (end 223.58 85.5) (width 0.75) (layer B.Cu) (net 16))
 (segment (start 210.92 82.55538) (end 210.92 81) (width 0.75) (layer B.Cu) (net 17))
 (segment (start 208.24538 85.23) (end 210.92 82.55538) (width 0.75) (layer B.Cu) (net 17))
 (segment (start 206.31 85.23) (end 208.24538 85.23) (width 0.75) (layer B.Cu) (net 17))
 (segment (start 206.31 85.23) (end 206.31 87.77) (width 0.75) (layer B.Cu) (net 17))
 (segment (start 209 77.5) (end 209 78) (width 1.25) (layer B.Cu) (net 18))
 (segment (start 209 78) (end 206.31 80.69) (width 1.25) (layer B.Cu) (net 18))
 (segment (start 206.31 80.69) (end 206.31 82.69) (width 1.25) (layer B.Cu) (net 18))
 (segment (start 210.46 62.5) (end 208.5 62.5) (width 1.25) (layer B.Cu) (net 18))
 (segment (start 208.5 62.5) (end 207 64) (width 1.25) (layer B.Cu) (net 18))
 (via (at 209 77.5) (size 1.25) (drill 0.5) (layers F.Cu B.Cu) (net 18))
 (segment (start 206.31 80.69) (end 209 78) (width 0.25) (layer B.Cu) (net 18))
 (segment (start 206.31 82.69) (end 206.31 80.69) (width 0.25) (layer B.Cu) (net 18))
 (segment (start 207 64) (end 208.5 62.5) (width 0.25) (layer B.Cu) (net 18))
 (via (at 207 64) (size 1.25) (drill 0.5) (layers F.Cu B.Cu) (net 18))
 (segment (start 209 66) (end 207 64) (width 0.25) (layer F.Cu) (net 18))
 (segment (start 209 77.5) (end 209 66) (width 0.25) (layer F.Cu) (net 18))
 (segment (start 210.5 66.5) (end 210.129821 66.870179) (width 0.75) (layer B.Cu) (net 18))
 (segment (start 210.129821 66.870179) (end 208.749881 66.870179) (width 0.75) (layer B.Cu) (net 18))
 (segment (start 208.749881 66.870179) (end 208.12006 67.5) (width 0.75) (layer B.Cu) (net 18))
 (segment (start 208.12006 67.5) (end 205.62 67.5) (width 0.75) (layer B.Cu) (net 18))
 (segment (start 210.5 63.04038) (end 210.5 66.5) (width 0.75) (layer B.Cu) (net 18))
 (segment (start 210.46 62.5) (end 210.46 63.00038) (width 0.75) (layer B.Cu) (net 18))
 (segment (start 210.46 63.00038) (end 210.5 63.04038) (width 0.75) (layer B.Cu) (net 18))
 (segment (start 206.31 82.69) (end 206.19 82.69) (width 0.75) (layer B.Cu) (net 18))
 (segment (start 204 67.5) (end 205.62 67.5) (width 0.75) (layer B.Cu) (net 18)))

